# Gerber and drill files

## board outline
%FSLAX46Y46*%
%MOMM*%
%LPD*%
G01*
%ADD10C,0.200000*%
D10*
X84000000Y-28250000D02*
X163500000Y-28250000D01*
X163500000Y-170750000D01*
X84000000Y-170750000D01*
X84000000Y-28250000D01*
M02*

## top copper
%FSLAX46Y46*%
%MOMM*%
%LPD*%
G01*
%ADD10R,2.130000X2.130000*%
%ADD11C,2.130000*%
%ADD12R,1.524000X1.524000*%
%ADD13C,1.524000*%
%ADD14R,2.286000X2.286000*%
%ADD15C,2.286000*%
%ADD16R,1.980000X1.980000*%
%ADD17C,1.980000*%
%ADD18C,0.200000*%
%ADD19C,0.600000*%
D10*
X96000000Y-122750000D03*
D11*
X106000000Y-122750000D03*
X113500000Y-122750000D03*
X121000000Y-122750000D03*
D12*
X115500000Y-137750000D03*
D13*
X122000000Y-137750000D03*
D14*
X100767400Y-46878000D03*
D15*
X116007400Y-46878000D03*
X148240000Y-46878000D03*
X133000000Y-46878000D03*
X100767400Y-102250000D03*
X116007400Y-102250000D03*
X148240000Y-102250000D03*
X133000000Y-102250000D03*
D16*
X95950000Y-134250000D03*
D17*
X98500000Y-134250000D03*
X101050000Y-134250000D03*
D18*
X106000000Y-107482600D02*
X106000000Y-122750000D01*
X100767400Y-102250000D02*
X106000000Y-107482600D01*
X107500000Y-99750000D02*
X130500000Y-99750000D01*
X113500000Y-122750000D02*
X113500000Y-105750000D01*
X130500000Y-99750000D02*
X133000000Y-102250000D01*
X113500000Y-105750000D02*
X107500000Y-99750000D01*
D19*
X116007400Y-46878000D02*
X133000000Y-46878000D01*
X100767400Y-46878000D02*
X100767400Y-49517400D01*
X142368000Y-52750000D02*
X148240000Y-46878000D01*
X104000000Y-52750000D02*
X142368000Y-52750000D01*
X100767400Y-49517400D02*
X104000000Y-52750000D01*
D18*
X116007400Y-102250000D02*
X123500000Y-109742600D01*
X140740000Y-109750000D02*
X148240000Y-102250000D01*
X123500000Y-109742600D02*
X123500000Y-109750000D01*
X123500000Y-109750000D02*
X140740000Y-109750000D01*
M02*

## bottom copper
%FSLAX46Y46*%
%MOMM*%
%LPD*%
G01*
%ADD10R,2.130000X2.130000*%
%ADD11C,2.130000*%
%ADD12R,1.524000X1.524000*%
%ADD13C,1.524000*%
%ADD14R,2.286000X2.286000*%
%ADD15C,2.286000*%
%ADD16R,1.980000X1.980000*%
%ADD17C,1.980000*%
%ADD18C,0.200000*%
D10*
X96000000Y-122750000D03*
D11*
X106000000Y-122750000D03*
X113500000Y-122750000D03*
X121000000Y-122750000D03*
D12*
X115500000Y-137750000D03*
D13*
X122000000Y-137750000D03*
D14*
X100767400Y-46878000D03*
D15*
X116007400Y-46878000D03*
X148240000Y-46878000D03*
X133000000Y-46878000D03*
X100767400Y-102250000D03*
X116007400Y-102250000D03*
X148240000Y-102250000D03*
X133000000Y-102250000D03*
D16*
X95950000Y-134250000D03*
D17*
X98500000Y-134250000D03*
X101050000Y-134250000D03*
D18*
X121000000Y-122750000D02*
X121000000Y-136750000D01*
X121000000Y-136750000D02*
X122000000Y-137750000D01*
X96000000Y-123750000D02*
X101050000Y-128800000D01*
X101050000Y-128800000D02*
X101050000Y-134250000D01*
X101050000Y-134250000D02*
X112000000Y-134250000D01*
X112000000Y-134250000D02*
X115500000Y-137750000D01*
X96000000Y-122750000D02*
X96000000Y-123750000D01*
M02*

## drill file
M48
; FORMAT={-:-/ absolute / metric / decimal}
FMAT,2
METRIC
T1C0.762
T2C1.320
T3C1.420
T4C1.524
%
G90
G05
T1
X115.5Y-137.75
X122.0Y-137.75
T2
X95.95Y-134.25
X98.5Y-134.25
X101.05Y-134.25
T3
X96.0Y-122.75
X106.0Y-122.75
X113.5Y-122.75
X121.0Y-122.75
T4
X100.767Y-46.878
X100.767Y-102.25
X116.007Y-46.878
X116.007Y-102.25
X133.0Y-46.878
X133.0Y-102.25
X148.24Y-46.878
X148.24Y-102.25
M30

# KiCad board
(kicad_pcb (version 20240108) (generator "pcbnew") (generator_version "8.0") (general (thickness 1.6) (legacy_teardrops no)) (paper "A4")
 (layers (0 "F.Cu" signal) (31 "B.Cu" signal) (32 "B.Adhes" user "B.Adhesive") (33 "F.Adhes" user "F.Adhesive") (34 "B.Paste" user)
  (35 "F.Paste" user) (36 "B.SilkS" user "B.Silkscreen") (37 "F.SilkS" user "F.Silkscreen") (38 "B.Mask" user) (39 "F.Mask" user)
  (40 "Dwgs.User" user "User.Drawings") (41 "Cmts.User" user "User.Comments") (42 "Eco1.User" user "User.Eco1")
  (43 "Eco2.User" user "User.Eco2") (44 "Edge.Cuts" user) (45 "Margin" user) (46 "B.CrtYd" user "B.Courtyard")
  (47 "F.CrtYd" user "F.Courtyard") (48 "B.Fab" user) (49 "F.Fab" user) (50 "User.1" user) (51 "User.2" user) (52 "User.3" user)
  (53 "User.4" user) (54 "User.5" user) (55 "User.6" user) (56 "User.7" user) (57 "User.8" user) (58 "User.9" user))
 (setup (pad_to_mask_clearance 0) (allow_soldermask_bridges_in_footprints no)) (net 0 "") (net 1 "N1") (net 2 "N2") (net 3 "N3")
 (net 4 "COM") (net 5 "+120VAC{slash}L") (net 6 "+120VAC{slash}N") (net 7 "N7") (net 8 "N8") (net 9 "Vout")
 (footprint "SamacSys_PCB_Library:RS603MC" (layer "F.Cu") (at 96 122.75)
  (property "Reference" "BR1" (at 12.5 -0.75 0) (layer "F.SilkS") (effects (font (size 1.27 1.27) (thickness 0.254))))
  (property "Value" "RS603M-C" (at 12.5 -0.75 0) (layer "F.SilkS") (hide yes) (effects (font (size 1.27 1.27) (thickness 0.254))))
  (pad "1" thru_hole rect (at 0 0 90) (size 2.13 2.13) (drill 1.42) (layers "*.Cu" "*.Mask" "F.SilkS") (remove_unused_layers no)
   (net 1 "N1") (thermal_bridge_angle 45))
  (pad "2" thru_hole circle (at 10 0 90) (size 2.13 2.13) (drill 1.42) (layers "*.Cu" "*.Mask" "F.SilkS") (remove_unused_layers no)
   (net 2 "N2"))
  (pad "3" thru_hole circle (at 17.5 0 90) (size 2.13 2.13) (drill 1.42) (layers "*.Cu" "*.Mask" "F.SilkS") (remove_unused_layers no)
   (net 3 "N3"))
  (pad "4" thru_hole circle (at 25 0 90) (size 2.13 2.13) (drill 1.42) (layers "*.Cu" "*.Mask" "F.SilkS") (remove_unused_layers no)
   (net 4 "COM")))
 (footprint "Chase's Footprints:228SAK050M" (layer "F.Cu") (at 118.75 137.75 180)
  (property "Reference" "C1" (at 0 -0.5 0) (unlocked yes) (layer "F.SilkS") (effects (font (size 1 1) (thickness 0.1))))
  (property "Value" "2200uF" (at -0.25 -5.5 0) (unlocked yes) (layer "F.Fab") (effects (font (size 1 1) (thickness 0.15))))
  (pad "1" thru_hole rect (at 3.25 0 180) (size 1.524 1.524) (drill 0.762) (layers "*.Cu" "*.Mask") (remove_unused_layers no) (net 1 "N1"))
  (pad "2" thru_hole circle (at -3.25 0 180) (size 1.524 1.524) (drill 0.762) (layers "*.Cu" "*.Mask") (remove_unused_layers no)
   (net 4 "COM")))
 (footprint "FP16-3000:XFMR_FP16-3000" (layer "F.Cu") (at 124.5037 74.564)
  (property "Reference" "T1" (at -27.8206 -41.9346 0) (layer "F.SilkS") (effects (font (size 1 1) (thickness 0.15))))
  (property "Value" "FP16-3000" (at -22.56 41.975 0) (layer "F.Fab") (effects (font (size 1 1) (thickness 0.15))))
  (pad "1" thru_hole rect (at -23.7363 -27.686) (size 2.286 2.286) (drill 1.524) (layers "*.Cu" "*.Mask") (remove_unused_layers no)
   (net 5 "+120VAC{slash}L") (solder_mask_margin 0.102))
  (pad "2" thru_hole circle (at -8.4963 -27.686) (size 2.286 2.286) (drill 1.524) (layers "*.Cu" "*.Mask") (remove_unused_layers no)
   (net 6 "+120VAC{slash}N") (solder_mask_margin 0.102))
  (pad "3" thru_hole circle (at 23.7363 -27.686) (size 2.286 2.286) (drill 1.524) (layers "*.Cu" "*.Mask") (remove_unused_layers no)
   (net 5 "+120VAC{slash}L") (solder_mask_margin 0.102))
  (pad "4" thru_hole circle (at 8.4963 -27.686) (size 2.286 2.286) (drill 1.524) (layers "*.Cu" "*.Mask") (remove_unused_layers no)
   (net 6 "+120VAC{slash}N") (solder_mask_margin 0.102))
  (pad "5" thru_hole circle (at -23.7363 27.686) (size 2.286 2.286) (drill 1.524) (layers "*.Cu" "*.Mask") (remove_unused_layers no)
   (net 2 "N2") (solder_mask_margin 0.102))
  (pad "6" thru_hole circle (at -8.4963 27.686) (size 2.286 2.286) (drill 1.524) (layers "*.Cu" "*.Mask") (remove_unused_layers no)
   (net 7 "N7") (solder_mask_margin 0.102))
  (pad "7" thru_hole circle (at 23.7363 27.686) (size 2.286 2.286) (drill 1.524) (layers "*.Cu" "*.Mask") (remove_unused_layers no)
   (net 7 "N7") (solder_mask_margin 0.102))
  (pad "8" thru_hole circle (at 8.4963 27.686) (size 2.286 2.286) (drill 1.524) (layers "*.Cu" "*.Mask") (remove_unused_layers no)
   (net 3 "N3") (solder_mask_margin 0.102)))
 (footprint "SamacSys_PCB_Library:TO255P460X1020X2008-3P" (layer "F.Cu") (at 95.95 134.25)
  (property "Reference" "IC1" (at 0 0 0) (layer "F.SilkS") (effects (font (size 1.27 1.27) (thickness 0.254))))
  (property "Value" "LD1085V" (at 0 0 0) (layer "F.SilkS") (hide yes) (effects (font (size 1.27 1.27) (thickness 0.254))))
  (pad "1" thru_hole rect (at 0 0 90) (size 1.98 1.98) (drill 1.32) (layers "*.Cu" "*.Mask" "F.SilkS") (remove_unused_layers no)
   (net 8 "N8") (thermal_bridge_angle 45))
  (pad "2" thru_hole circle (at 2.55 0 90) (size 1.98 1.98) (drill 1.32) (layers "*.Cu" "*.Mask" "F.SilkS") (remove_unused_layers no)
   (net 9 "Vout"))
  (pad "3" thru_hole circle (at 5.1 0 90) (size 1.98 1.98) (drill 1.32) (layers "*.Cu" "*.Mask" "F.SilkS") (remove_unused_layers no)
   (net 1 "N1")))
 (gr_rect (start 84 28.25) (end 163.5 170.75) (stroke (width 0.2) (type default)) (fill none) (layer "Edge.Cuts"))
 (segment (start 106 107.4826) (end 106 122.75) (width 0.2) (layer "F.Cu") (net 2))
 (segment (start 100.7674 102.25) (end 106 107.4826) (width 0.2) (layer "F.Cu") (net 2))
 (segment (start 121 122.75) (end 121 136.75) (width 0.2) (layer "B.Cu") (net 4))
 (segment (start 121 136.75) (end 122 137.75) (width 0.2) (layer "B.Cu") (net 4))
 (segment (start 107.5 99.75) (end 130.5 99.75) (width 0.2) (layer "F.Cu") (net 3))
 (segment (start 113.5 122.75) (end 113.5 105.75) (width 0.2) (layer "F.Cu") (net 3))
 (segment (start 130.5 99.75) (end 133 102.25) (width 0.2) (layer "F.Cu") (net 3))
 (segment (start 113.5 105.75) (end 107.5 99.75) (width 0.2) (layer "F.Cu") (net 3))
 (segment (start 96 123.75) (end 101.05 128.8) (width 0.2) (layer "B.Cu") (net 1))
 (segment (start 101.05 128.8) (end 101.05 134.25) (width 0.2) (layer "B.Cu") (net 1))
 (segment (start 101.05 134.25) (end 112 134.25) (width 0.2) (layer "B.Cu") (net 1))
 (segment (start 112 134.25) (end 115.5 137.75) (width 0.2) (layer "B.Cu") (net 1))
 (segment (start 96 122.75) (end 96 123.75) (width 0.2) (layer "B.Cu") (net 1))
 (segment (start 116.0074 46.878) (end 133 46.878) (width 0.6) (layer "F.Cu") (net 6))
 (segment (start 100.7674 46.878) (end 100.7674 49.5174) (width 0.6) (layer "F.Cu") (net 5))
 (segment (start 142.368 52.75) (end 148.24 46.878) (width 0.6) (layer "F.Cu") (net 5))
 (segment (start 104 52.75) (end 142.368 52.75) (width 0.6) (layer "F.Cu") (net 5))
 (segment (start 100.7674 49.5174) (end 104 52.75) (width 0.6) (layer "F.Cu") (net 5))
 (segment (start 116.0074 102.25) (end 123.5 109.7426) (width 0.2) (layer "F.Cu") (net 7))
 (segment (start 140.74 109.75) (end 148.24 102.25) (width 0.2) (layer "F.Cu") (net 7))
 (segment (start 123.5 109.7426) (end 123.5 109.75) (width 0.2) (layer "F.Cu") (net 7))
 (segment (start 123.5 109.75) (end 140.74 109.75) (width 0.2) (layer "F.Cu") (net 7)))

